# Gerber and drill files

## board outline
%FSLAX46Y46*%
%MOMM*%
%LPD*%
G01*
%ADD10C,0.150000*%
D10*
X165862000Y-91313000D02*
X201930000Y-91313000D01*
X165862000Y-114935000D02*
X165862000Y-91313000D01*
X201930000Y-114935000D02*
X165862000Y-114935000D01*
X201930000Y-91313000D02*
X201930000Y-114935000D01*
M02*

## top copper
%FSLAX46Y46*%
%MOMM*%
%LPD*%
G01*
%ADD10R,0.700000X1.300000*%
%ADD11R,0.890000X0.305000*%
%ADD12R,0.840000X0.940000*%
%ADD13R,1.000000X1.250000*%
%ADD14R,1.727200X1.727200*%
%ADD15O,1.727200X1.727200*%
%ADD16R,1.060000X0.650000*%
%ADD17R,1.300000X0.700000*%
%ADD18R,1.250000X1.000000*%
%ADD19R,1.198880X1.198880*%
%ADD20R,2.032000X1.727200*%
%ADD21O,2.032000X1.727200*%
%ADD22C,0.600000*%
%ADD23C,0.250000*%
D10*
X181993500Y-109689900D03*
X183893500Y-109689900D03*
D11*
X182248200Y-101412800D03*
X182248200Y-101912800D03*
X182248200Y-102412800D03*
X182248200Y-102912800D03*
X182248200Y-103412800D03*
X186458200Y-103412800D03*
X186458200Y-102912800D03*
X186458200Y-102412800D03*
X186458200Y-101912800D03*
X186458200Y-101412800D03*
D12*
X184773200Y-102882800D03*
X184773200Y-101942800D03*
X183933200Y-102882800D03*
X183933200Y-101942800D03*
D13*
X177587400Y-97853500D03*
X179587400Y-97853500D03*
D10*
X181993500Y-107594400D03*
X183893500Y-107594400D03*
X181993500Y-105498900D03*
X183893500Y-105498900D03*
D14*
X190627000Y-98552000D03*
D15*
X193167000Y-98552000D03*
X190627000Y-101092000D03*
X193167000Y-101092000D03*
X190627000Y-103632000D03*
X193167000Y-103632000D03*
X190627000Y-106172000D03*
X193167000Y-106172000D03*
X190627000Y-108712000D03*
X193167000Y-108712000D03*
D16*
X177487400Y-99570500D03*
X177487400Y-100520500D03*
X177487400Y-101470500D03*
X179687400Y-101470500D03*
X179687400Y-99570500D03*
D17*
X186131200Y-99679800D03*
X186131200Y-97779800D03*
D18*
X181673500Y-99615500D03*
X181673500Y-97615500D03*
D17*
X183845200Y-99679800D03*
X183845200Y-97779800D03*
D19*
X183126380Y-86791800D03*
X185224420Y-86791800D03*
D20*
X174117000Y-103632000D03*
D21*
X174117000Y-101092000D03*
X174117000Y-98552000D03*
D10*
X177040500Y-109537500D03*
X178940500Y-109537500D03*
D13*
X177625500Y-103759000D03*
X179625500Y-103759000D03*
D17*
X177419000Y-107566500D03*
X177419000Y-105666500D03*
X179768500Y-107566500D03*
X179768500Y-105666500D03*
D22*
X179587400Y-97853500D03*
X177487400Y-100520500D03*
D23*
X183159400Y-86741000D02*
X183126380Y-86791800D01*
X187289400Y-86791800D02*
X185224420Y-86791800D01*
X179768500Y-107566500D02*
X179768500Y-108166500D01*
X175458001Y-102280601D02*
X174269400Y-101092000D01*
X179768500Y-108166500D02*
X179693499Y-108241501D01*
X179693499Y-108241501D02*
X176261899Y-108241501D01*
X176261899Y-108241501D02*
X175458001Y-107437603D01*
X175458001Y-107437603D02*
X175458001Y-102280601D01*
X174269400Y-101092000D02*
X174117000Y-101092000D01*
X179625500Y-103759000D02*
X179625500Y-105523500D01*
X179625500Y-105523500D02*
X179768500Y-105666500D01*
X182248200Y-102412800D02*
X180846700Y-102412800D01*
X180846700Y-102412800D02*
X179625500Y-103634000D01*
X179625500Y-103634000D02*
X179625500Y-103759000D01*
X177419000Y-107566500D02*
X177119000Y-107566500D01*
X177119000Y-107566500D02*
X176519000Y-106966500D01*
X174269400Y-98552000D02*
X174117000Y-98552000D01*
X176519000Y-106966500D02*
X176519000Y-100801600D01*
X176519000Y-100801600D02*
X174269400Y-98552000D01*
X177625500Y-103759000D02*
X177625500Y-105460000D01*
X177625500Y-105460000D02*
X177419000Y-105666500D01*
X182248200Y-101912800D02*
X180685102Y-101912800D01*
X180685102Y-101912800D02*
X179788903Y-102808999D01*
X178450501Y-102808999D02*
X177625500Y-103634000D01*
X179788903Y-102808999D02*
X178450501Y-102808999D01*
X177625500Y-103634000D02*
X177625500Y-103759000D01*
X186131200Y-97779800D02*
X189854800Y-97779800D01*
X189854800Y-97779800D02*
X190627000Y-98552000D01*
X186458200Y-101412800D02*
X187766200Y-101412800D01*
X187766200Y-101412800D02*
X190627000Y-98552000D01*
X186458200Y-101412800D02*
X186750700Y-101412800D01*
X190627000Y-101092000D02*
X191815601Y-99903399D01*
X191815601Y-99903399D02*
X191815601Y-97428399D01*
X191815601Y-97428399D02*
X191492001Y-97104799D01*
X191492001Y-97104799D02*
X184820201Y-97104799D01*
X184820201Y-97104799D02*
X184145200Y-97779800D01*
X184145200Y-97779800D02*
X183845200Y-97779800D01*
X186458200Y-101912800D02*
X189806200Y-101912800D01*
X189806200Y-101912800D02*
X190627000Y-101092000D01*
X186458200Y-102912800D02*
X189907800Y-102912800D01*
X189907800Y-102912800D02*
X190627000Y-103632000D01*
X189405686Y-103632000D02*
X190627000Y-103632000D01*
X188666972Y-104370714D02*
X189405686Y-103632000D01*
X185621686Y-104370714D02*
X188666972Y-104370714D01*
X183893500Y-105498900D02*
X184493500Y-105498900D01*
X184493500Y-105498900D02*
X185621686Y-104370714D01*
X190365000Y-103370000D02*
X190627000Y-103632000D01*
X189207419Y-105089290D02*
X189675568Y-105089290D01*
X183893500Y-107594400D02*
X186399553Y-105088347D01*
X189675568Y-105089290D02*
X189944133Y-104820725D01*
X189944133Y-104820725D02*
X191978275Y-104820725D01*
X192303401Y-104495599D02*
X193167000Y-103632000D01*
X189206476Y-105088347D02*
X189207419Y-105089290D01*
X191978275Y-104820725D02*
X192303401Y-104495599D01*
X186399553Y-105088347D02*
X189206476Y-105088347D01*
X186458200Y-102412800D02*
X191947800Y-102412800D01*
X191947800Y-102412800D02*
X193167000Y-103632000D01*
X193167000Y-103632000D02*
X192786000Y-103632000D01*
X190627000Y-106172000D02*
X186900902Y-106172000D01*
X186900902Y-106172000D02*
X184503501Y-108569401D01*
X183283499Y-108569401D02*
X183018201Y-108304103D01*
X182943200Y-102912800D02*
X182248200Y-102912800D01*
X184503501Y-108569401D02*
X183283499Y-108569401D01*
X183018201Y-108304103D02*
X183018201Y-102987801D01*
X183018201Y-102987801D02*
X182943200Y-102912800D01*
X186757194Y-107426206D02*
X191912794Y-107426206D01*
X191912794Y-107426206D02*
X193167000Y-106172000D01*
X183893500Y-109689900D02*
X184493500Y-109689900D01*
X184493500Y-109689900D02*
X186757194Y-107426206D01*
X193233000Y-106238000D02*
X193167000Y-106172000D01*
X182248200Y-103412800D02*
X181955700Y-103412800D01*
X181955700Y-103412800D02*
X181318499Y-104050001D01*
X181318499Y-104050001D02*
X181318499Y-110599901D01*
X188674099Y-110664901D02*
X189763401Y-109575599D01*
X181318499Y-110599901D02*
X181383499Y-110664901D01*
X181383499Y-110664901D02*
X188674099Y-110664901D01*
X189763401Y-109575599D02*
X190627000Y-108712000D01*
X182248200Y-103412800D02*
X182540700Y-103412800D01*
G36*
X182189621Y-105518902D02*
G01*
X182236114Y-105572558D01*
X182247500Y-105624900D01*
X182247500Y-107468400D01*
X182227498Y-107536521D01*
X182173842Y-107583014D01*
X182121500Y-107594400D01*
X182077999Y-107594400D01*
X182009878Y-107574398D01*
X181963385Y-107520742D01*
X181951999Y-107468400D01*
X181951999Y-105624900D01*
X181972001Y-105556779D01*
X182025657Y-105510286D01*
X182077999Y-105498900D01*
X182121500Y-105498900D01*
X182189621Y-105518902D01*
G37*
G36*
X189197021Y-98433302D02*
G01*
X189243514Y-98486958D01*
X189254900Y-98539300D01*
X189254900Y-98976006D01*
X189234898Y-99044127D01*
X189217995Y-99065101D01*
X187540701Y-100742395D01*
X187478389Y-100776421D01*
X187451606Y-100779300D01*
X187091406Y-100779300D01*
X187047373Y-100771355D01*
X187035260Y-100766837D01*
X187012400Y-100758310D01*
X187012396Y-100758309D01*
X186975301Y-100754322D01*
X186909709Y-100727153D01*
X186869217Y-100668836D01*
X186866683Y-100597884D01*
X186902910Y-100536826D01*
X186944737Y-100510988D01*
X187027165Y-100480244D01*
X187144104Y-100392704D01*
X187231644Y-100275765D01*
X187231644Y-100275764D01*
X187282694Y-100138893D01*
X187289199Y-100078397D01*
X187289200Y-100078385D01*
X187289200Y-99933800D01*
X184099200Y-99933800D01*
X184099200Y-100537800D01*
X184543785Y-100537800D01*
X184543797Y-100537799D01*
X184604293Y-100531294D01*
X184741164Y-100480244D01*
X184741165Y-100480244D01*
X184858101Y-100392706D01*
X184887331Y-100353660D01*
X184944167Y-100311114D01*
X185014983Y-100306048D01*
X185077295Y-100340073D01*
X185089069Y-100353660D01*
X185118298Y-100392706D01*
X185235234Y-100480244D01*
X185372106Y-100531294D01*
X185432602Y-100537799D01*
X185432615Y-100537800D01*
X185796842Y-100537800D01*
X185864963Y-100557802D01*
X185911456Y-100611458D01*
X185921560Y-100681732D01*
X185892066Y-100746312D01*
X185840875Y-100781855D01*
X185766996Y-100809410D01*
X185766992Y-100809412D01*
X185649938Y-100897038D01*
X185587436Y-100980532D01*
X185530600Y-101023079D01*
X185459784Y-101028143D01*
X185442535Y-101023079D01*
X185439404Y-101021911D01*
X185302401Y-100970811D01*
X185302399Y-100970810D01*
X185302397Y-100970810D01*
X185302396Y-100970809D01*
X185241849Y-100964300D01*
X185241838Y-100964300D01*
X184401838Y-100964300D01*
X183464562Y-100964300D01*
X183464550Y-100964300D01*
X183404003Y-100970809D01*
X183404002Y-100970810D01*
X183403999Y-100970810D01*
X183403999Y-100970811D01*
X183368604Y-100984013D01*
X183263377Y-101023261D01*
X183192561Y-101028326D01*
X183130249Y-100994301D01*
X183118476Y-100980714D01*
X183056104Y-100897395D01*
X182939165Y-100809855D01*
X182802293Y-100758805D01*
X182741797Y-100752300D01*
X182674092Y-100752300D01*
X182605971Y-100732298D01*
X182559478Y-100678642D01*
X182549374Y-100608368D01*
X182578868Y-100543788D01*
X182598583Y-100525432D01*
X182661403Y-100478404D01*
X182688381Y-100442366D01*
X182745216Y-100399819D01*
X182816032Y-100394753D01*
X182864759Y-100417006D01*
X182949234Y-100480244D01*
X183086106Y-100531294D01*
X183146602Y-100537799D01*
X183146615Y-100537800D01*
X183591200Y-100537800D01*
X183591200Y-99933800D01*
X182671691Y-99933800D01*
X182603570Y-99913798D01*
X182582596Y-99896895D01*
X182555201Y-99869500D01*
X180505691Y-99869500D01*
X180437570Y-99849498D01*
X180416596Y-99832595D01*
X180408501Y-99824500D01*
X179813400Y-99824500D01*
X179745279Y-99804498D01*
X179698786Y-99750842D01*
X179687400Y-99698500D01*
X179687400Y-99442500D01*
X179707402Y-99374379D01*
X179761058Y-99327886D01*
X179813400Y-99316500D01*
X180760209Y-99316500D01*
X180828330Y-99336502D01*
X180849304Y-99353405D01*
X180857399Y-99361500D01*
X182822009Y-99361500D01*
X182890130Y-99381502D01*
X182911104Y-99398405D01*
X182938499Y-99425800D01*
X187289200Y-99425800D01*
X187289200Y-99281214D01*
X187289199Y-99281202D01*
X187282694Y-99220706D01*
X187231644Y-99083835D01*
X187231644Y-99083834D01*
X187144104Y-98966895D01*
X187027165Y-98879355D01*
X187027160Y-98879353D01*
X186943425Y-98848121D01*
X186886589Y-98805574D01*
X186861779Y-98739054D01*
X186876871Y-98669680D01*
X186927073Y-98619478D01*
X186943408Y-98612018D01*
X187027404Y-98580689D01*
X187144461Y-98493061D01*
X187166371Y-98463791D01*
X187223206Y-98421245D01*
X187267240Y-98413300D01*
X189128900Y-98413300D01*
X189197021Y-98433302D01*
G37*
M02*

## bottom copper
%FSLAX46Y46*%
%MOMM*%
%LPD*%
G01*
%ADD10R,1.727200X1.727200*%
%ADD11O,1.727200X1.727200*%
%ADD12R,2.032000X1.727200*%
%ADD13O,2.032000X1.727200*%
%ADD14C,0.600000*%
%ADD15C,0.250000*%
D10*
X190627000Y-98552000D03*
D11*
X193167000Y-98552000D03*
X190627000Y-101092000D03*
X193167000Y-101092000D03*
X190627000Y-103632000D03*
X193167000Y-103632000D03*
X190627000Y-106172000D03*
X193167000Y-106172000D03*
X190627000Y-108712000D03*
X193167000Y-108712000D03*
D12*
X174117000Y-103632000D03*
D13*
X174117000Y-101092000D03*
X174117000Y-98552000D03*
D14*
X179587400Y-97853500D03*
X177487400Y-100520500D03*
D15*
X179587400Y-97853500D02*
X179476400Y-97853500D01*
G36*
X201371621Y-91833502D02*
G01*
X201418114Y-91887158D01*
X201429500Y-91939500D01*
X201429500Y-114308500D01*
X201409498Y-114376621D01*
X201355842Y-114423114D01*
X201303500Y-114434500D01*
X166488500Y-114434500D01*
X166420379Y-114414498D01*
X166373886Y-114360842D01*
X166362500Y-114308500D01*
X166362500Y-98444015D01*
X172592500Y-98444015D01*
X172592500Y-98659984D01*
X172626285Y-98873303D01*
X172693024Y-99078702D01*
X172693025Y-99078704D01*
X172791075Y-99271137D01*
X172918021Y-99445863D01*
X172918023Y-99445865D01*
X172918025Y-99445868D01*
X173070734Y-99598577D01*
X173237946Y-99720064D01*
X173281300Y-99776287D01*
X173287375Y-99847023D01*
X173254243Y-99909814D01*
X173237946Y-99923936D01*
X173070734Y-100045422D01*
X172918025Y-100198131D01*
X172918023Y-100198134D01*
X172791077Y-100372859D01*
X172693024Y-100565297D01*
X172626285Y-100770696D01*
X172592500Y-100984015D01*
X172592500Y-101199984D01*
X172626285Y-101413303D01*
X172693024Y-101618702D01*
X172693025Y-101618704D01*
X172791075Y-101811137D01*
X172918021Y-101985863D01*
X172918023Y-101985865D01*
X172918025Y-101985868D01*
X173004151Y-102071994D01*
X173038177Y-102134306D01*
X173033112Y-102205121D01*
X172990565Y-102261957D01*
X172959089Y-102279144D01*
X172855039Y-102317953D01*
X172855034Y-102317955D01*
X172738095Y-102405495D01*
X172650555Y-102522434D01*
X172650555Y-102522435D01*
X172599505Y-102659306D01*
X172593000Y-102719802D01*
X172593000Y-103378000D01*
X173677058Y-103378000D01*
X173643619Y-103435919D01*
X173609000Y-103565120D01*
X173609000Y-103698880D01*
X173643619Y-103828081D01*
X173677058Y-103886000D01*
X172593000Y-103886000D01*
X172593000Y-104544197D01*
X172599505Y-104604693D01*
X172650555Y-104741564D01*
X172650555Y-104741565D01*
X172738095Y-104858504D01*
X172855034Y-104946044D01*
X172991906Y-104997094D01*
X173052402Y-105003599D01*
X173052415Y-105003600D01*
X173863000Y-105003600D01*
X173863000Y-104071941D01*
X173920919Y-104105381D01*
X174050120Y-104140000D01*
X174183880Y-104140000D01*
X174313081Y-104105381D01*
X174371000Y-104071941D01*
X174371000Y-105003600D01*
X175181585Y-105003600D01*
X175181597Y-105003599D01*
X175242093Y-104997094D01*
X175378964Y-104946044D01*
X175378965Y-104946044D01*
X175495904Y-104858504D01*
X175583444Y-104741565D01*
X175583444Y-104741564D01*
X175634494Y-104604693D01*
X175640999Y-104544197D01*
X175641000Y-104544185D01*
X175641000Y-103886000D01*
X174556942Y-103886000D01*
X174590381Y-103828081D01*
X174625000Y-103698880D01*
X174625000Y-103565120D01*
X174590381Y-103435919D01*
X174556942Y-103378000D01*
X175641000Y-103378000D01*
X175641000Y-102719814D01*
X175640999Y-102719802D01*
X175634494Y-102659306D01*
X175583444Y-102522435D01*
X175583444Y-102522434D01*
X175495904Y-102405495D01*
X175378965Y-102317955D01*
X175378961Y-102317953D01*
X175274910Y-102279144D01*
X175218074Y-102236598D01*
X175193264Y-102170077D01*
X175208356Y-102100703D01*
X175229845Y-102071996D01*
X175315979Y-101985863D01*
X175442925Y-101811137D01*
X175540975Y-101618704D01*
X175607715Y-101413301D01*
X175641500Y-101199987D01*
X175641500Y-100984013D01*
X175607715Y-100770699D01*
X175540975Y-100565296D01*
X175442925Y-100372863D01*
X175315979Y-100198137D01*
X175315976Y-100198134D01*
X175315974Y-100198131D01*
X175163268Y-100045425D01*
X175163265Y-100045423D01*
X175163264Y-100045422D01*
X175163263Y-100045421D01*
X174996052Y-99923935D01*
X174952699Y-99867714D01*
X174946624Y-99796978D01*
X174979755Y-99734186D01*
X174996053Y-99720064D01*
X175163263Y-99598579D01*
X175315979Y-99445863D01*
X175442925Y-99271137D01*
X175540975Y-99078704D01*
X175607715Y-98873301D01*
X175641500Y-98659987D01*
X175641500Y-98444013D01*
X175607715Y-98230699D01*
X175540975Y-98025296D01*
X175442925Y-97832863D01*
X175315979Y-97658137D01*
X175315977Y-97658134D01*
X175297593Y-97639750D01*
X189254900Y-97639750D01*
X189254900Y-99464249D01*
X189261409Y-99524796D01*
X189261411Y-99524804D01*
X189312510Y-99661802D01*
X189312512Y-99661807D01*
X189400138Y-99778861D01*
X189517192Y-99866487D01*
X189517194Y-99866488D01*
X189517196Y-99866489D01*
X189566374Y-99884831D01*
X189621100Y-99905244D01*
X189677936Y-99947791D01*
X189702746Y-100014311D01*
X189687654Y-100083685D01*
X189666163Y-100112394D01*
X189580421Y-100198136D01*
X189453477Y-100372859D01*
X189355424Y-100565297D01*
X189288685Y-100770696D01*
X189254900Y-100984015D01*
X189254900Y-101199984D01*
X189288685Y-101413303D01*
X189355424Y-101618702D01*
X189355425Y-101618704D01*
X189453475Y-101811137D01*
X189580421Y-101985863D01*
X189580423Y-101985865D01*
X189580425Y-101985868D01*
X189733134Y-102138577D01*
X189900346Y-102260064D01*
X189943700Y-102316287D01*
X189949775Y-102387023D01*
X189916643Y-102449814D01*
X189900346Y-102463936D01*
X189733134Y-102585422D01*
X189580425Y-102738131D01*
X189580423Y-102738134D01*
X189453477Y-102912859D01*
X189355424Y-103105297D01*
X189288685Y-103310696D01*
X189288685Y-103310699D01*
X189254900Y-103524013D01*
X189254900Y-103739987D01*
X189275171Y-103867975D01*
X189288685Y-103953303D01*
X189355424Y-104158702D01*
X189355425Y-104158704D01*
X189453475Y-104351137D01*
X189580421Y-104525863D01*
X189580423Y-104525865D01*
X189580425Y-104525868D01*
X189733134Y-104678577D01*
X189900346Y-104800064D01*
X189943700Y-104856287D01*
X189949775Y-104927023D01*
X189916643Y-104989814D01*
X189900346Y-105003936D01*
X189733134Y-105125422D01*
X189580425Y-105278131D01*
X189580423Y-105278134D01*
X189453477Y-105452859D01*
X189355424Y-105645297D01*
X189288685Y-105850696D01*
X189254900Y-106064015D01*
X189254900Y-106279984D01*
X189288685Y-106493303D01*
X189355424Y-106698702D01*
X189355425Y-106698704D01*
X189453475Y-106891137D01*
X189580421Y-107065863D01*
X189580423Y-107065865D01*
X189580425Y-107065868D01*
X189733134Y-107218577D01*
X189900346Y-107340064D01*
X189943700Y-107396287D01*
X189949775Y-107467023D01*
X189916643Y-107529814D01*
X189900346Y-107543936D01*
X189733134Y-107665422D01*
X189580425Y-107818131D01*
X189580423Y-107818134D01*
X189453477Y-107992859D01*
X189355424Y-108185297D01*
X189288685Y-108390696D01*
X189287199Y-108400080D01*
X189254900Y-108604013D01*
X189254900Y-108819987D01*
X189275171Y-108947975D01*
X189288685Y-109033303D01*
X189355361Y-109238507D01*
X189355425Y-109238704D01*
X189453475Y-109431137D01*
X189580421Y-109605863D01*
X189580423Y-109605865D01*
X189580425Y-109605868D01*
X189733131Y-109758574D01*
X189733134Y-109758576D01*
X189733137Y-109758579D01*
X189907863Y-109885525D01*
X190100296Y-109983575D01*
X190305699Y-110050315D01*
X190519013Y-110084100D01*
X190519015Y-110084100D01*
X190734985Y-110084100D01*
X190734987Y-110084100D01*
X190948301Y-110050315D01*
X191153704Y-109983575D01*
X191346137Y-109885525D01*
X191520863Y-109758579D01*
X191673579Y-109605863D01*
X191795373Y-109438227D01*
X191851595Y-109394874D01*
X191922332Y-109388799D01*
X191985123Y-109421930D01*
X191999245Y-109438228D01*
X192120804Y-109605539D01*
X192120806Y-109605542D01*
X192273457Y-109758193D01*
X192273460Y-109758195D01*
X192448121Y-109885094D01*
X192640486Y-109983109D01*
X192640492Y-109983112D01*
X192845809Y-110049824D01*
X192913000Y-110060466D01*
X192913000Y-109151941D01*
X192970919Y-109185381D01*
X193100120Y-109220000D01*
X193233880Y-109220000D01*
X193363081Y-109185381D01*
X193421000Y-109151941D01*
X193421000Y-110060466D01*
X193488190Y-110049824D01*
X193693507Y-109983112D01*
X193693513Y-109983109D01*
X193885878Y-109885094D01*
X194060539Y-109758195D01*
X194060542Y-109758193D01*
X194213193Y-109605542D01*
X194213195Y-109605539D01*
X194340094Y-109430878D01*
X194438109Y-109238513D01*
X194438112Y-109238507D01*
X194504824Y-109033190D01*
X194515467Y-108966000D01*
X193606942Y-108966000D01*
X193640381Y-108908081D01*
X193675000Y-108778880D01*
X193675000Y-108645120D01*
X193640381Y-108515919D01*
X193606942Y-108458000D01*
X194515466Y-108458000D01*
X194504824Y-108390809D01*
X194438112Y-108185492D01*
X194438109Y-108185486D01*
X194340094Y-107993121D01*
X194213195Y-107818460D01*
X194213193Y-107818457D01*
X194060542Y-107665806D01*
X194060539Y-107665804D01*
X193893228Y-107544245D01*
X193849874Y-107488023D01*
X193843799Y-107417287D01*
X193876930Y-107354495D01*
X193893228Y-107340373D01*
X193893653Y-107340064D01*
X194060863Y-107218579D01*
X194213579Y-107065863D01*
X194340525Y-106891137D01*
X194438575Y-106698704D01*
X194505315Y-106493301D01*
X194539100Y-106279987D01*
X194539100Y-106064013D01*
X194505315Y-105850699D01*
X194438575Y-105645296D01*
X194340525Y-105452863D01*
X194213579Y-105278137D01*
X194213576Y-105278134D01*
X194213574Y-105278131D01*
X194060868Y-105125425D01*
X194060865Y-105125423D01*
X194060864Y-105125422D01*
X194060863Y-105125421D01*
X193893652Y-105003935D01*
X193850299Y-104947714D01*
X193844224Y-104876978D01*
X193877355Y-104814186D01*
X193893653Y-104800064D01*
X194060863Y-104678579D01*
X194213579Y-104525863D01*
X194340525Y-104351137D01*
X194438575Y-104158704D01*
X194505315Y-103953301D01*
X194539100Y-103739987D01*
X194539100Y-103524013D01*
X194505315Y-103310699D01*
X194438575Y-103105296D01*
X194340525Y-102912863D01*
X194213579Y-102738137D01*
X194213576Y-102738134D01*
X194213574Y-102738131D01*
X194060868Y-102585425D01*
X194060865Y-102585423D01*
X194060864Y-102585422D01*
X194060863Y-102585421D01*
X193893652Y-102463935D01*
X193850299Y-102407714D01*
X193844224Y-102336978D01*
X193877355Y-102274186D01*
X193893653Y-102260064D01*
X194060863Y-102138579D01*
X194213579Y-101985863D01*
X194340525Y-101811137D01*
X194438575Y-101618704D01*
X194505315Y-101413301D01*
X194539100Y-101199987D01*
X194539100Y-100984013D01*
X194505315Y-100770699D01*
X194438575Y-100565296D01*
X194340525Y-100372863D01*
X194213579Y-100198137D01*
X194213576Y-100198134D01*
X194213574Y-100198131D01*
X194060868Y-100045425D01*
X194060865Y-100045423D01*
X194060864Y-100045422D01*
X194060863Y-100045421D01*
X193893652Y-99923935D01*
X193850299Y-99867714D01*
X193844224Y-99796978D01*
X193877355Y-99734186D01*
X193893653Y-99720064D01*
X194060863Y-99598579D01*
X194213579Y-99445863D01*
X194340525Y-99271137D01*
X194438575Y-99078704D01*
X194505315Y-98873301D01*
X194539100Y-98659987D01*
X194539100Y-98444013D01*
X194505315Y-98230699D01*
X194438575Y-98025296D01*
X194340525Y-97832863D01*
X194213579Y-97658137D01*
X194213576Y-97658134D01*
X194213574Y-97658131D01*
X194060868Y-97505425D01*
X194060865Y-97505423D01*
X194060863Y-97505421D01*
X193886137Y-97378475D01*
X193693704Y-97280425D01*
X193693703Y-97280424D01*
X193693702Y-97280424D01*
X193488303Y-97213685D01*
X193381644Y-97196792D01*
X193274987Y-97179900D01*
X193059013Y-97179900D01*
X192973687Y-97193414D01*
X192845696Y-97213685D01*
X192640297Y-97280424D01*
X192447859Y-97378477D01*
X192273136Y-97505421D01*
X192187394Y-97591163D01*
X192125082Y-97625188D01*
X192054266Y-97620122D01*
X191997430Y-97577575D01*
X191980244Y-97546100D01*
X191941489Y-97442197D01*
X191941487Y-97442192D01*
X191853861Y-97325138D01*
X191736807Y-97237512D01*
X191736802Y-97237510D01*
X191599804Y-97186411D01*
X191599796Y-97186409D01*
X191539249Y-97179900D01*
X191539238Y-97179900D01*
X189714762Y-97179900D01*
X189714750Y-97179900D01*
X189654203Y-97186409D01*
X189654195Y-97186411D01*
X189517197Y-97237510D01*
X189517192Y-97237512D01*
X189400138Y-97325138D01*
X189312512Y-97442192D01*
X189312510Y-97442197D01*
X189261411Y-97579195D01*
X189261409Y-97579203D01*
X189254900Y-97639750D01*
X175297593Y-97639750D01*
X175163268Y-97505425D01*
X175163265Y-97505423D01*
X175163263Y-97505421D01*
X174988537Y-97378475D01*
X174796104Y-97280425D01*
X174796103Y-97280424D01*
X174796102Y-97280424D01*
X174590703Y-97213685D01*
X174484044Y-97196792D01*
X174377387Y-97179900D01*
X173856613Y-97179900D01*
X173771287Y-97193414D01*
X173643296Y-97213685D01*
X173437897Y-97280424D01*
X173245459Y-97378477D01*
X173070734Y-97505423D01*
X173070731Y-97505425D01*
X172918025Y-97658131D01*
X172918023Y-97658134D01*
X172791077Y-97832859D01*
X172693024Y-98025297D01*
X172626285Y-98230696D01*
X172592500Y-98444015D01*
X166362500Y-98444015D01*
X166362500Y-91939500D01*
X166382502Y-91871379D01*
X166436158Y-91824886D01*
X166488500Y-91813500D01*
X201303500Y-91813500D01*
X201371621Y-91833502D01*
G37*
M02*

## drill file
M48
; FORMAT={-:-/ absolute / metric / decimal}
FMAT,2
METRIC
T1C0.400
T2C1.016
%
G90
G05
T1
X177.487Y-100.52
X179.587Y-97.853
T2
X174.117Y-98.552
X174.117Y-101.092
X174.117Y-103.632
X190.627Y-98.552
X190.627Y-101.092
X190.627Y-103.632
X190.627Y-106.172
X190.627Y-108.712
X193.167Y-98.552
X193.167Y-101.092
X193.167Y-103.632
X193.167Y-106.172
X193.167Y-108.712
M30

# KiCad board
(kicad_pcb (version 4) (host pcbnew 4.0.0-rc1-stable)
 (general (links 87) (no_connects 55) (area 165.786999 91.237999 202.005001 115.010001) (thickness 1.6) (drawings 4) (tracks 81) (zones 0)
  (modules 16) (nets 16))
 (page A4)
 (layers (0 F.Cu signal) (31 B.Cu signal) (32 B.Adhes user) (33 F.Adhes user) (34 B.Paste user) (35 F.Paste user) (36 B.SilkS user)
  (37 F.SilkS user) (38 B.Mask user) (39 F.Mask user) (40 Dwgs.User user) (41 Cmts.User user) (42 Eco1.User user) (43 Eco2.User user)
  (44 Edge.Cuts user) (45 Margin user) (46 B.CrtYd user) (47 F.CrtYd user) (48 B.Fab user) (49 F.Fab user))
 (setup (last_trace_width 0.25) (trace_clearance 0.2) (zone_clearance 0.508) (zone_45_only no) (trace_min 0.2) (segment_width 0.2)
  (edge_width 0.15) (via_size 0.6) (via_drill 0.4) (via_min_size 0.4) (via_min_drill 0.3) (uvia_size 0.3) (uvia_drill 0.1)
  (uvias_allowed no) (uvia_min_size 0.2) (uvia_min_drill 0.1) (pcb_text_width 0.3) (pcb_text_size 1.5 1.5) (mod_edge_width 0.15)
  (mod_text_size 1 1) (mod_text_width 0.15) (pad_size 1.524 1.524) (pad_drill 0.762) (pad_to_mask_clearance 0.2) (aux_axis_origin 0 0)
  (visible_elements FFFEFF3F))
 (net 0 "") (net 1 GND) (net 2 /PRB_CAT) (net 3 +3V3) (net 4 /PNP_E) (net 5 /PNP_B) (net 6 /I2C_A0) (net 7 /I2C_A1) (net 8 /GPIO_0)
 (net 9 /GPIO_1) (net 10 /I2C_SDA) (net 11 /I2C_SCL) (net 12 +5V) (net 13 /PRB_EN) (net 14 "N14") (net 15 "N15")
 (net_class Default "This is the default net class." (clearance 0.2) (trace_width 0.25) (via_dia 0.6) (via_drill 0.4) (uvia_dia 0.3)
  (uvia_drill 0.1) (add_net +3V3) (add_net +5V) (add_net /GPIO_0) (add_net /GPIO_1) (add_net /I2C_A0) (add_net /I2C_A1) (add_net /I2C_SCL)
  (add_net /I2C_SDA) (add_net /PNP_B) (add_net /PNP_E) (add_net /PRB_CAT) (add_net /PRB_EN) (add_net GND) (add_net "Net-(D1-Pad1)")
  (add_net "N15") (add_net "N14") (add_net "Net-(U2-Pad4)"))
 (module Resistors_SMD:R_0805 (layer F.Cu) (at 182.9435 109.6899)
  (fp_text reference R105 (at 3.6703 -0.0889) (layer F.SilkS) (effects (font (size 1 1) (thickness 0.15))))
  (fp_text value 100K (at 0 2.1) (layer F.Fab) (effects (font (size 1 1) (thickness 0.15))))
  (pad 1 smd rect (at -0.95 0) (size 0.7 1.3) (layers F.Cu F.Paste F.Mask) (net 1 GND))
  (pad 2 smd rect (at 0.95 0) (size 0.7 1.3) (layers F.Cu F.Paste F.Mask) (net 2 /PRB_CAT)))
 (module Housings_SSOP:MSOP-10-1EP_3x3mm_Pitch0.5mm (layer F.Cu) (at 184.3532 102.4128)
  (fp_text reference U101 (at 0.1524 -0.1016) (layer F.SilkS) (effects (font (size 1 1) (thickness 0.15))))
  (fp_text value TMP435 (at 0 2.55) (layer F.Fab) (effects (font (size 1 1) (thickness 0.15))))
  (pad 1 smd rect (at -2.105 -1) (size 0.89 0.305) (layers F.Cu F.Paste F.Mask) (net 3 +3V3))
  (pad 2 smd rect (at -2.105 -0.5) (size 0.89 0.305) (layers F.Cu F.Paste F.Mask) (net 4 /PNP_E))
  (pad 3 smd rect (at -2.105 0) (size 0.89 0.305) (layers F.Cu F.Paste F.Mask) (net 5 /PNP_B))
  (pad 4 smd rect (at -2.105 0.5) (size 0.89 0.305) (layers F.Cu F.Paste F.Mask) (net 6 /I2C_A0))
  (pad 5 smd rect (at -2.105 1) (size 0.89 0.305) (layers F.Cu F.Paste F.Mask) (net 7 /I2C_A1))
  (pad 6 smd rect (at 2.105 1) (size 0.89 0.305) (layers F.Cu F.Paste F.Mask) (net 1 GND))
  (pad 7 smd rect (at 2.105 0.5) (size 0.89 0.305) (layers F.Cu F.Paste F.Mask) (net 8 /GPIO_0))
  (pad 8 smd rect (at 2.105 0) (size 0.89 0.305) (layers F.Cu F.Paste F.Mask) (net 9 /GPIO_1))
  (pad 9 smd rect (at 2.105 -0.5) (size 0.89 0.305) (layers F.Cu F.Paste F.Mask) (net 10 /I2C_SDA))
  (pad 10 smd rect (at 2.105 -1) (size 0.89 0.305) (layers F.Cu F.Paste F.Mask) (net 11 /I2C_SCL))
  (pad 11 smd rect (at 0.42 0.47) (size 0.84 0.94) (layers F.Cu F.Paste F.Mask) (solder_paste_margin_ratio -0.2))
  (pad 11 smd rect (at 0.42 -0.47) (size 0.84 0.94) (layers F.Cu F.Paste F.Mask) (solder_paste_margin_ratio -0.2))
  (pad 11 smd rect (at -0.42 0.47) (size 0.84 0.94) (layers F.Cu F.Paste F.Mask) (solder_paste_margin_ratio -0.2))
  (pad 11 smd rect (at -0.42 -0.47) (size 0.84 0.94) (layers F.Cu F.Paste F.Mask) (solder_paste_margin_ratio -0.2)))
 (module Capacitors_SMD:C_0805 (layer F.Cu) (at 178.5874 97.8535)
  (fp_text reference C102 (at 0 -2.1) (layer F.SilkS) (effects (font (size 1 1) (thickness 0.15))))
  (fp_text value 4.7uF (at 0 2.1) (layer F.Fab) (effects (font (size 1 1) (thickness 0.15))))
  (pad 1 smd rect (at -1 0) (size 1 1.25) (layers F.Cu F.Paste F.Mask) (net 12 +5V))
  (pad 2 smd rect (at 1 0) (size 1 1.25) (layers F.Cu F.Paste F.Mask) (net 1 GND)))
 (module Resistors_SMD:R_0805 (layer F.Cu) (at 182.9435 107.5944)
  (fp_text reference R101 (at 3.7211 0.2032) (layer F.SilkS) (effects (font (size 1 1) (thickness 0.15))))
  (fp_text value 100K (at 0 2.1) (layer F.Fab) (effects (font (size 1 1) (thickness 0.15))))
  (pad 1 smd rect (at -0.95 0) (size 0.7 1.3) (layers F.Cu F.Paste F.Mask) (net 3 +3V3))
  (pad 2 smd rect (at 0.95 0) (size 0.7 1.3) (layers F.Cu F.Paste F.Mask) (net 9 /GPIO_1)))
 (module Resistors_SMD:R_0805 (layer F.Cu) (at 182.9435 105.4989)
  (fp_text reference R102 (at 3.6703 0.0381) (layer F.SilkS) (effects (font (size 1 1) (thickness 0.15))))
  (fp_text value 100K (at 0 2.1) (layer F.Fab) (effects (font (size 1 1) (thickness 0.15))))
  (pad 1 smd rect (at -0.95 0) (size 0.7 1.3) (layers F.Cu F.Paste F.Mask) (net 3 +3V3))
  (pad 2 smd rect (at 0.95 0) (size 0.7 1.3) (layers F.Cu F.Paste F.Mask) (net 8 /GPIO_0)))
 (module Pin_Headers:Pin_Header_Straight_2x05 (layer F.Cu) (at 190.627 98.552)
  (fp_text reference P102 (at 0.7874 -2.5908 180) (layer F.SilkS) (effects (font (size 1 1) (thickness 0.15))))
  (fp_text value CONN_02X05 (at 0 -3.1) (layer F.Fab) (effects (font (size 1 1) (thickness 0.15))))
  (pad 1 thru_hole rect (at 0 0) (size 1.7272 1.7272) (drill 1.016) (layers *.Cu *.Mask F.SilkS) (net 11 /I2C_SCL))
  (pad 2 thru_hole oval (at 2.54 0) (size 1.7272 1.7272) (drill 1.016) (layers *.Cu *.Mask F.SilkS) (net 12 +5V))
  (pad 3 thru_hole oval (at 0 2.54) (size 1.7272 1.7272) (drill 1.016) (layers *.Cu *.Mask F.SilkS) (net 10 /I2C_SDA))
  (pad 4 thru_hole oval (at 2.54 2.54) (size 1.7272 1.7272) (drill 1.016) (layers *.Cu *.Mask F.SilkS) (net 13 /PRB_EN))
  (pad 5 thru_hole oval (at 0 5.08) (size 1.7272 1.7272) (drill 1.016) (layers *.Cu *.Mask F.SilkS) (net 8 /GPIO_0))
  (pad 6 thru_hole oval (at 2.54 5.08) (size 1.7272 1.7272) (drill 1.016) (layers *.Cu *.Mask F.SilkS) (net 9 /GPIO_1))
  (pad 7 thru_hole oval (at 0 7.62) (size 1.7272 1.7272) (drill 1.016) (layers *.Cu *.Mask F.SilkS) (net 6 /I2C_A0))
  (pad 8 thru_hole oval (at 2.54 7.62) (size 1.7272 1.7272) (drill 1.016) (layers *.Cu *.Mask F.SilkS) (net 2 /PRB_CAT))
  (pad 9 thru_hole oval (at 0 10.16) (size 1.7272 1.7272) (drill 1.016) (layers *.Cu *.Mask F.SilkS) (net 7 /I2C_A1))
  (pad 10 thru_hole oval (at 2.54 10.16) (size 1.7272 1.7272) (drill 1.016) (layers *.Cu *.Mask F.SilkS) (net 1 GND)))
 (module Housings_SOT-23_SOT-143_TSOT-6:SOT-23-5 (layer F.Cu) (at 178.5874 100.5205)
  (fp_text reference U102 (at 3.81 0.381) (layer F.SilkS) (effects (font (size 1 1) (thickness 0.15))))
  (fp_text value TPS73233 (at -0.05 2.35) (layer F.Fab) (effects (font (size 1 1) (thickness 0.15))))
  (pad 1 smd rect (at -1.1 -0.95) (size 1.06 0.65) (layers F.Cu F.Paste F.Mask) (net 12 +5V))
  (pad 2 smd rect (at -1.1 0) (size 1.06 0.65) (layers F.Cu F.Paste F.Mask) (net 1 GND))
  (pad 3 smd rect (at -1.1 0.95) (size 1.06 0.65) (layers F.Cu F.Paste F.Mask) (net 13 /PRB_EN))
  (pad 4 smd rect (at 1.1 0.95) (size 1.06 0.65) (layers F.Cu F.Paste F.Mask) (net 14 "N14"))
  (pad 5 smd rect (at 1.1 -0.95) (size 1.06 0.65) (layers F.Cu F.Paste F.Mask) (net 3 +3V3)))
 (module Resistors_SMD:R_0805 (layer F.Cu) (at 186.1312 98.7298 90)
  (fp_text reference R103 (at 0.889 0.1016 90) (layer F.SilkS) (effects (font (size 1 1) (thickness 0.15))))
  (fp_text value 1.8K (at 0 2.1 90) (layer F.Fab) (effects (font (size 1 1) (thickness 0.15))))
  (pad 1 smd rect (at -0.95 0 90) (size 0.7 1.3) (layers F.Cu F.Paste F.Mask) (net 3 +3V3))
  (pad 2 smd rect (at 0.95 0 90) (size 0.7 1.3) (layers F.Cu F.Paste F.Mask) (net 11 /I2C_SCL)))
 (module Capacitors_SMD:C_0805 (layer F.Cu) (at 181.6735 98.6155 90)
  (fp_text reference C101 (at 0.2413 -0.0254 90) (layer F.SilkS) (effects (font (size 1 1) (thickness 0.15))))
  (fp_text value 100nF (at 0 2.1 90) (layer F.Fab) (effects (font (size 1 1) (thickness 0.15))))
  (pad 1 smd rect (at -1 0 90) (size 1 1.25) (layers F.Cu F.Paste F.Mask) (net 3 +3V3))
  (pad 2 smd rect (at 1 0 90) (size 1 1.25) (layers F.Cu F.Paste F.Mask) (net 1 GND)))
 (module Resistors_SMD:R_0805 (layer F.Cu) (at 183.8452 98.7298 90)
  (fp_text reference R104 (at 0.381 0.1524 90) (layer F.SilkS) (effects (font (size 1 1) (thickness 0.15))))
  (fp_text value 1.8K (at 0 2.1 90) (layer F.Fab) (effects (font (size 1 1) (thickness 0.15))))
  (pad 1 smd rect (at -0.95 0 90) (size 0.7 1.3) (layers F.Cu F.Paste F.Mask) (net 3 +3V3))
  (pad 2 smd rect (at 0.95 0 90) (size 0.7 1.3) (layers F.Cu F.Paste F.Mask) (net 10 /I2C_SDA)))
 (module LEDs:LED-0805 (layer F.Cu) (at 184.1754 86.7918 180)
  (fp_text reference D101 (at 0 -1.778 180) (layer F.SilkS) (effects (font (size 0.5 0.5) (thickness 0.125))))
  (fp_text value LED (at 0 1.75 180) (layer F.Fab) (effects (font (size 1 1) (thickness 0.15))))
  (pad 2 smd rect (at 1.04902 0) (size 1.19888 1.19888) (layers F.Cu F.Paste F.Mask) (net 3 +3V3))
  (pad 1 smd rect (at -1.04902 0) (size 1.19888 1.19888) (layers F.Cu F.Paste F.Mask) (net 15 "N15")))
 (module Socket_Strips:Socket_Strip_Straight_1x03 (layer F.Cu) (at 174.117 103.632 90)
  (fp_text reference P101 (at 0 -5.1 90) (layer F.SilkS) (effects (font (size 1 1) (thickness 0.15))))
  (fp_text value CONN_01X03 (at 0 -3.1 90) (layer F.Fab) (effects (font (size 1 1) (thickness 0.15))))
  (pad 1 thru_hole rect (at 0 0 90) (size 1.7272 2.032) (drill 1.016) (layers *.Cu *.Mask F.SilkS) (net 1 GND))
  (pad 2 thru_hole oval (at 2.54 0 90) (size 1.7272 2.032) (drill 1.016) (layers *.Cu *.Mask F.SilkS) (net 5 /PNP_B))
  (pad 3 thru_hole oval (at 5.08 0 90) (size 1.7272 2.032) (drill 1.016) (layers *.Cu *.Mask F.SilkS) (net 4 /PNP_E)))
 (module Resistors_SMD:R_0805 (layer F.Cu) (at 177.9905 109.5375)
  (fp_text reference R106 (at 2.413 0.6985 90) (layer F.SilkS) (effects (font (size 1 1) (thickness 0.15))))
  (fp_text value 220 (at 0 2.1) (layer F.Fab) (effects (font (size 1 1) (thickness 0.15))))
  (pad 1 smd rect (at -0.95 0) (size 0.7 1.3) (layers F.Cu F.Paste F.Mask) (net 15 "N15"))
  (pad 2 smd rect (at 0.95 0) (size 0.7 1.3) (layers F.Cu F.Paste F.Mask) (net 1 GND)))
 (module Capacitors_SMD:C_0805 (layer F.Cu) (at 178.6255 103.759)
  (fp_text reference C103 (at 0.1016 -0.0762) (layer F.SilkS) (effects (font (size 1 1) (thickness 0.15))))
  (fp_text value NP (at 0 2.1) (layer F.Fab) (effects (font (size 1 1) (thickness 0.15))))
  (pad 1 smd rect (at -1 0) (size 1 1.25) (layers F.Cu F.Paste F.Mask) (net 4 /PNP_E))
  (pad 2 smd rect (at 1 0) (size 1 1.25) (layers F.Cu F.Paste F.Mask) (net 5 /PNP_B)))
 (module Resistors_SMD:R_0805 (layer F.Cu) (at 177.419 106.6165 90)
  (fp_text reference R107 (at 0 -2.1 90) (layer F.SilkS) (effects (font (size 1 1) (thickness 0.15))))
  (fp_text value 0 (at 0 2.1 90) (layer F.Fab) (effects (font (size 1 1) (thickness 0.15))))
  (pad 1 smd rect (at -0.95 0 90) (size 0.7 1.3) (layers F.Cu F.Paste F.Mask) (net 4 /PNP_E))
  (pad 2 smd rect (at 0.95 0 90) (size 0.7 1.3) (layers F.Cu F.Paste F.Mask) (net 4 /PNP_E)))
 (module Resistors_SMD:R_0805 (layer F.Cu) (at 179.7685 106.6165 90)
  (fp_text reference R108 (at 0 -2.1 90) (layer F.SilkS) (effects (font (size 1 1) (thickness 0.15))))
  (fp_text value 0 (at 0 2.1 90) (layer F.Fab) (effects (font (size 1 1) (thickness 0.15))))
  (pad 1 smd rect (at -0.95 0 90) (size 0.7 1.3) (layers F.Cu F.Paste F.Mask) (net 5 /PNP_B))
  (pad 2 smd rect (at 0.95 0 90) (size 0.7 1.3) (layers F.Cu F.Paste F.Mask) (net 5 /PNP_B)))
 (gr_line (start 165.862 91.313) (end 201.93 91.313) (angle 90) (layer Edge.Cuts) (width 0.15))
 (gr_line (start 165.862 114.935) (end 165.862 91.313) (angle 90) (layer Edge.Cuts) (width 0.15))
 (gr_line (start 201.93 114.935) (end 165.862 114.935) (angle 90) (layer Edge.Cuts) (width 0.15))
 (gr_line (start 201.93 91.313) (end 201.93 114.935) (angle 90) (layer Edge.Cuts) (width 0.15))
 (segment (start 183.1594 86.741) (end 183.12638 86.7918) (width 0.25) (layer F.Cu) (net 3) (status 80000))
 (via (at 179.5874 97.8535) (size 0.6) (drill 0.4) (layers F.Cu B.Cu) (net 1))
 (via (at 177.4874 100.5205) (size 0.6) (drill 0.4) (layers F.Cu B.Cu) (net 1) (status 30))
 (segment (start 179.5874 97.8535) (end 179.4764 97.8535) (width 0.25) (layer B.Cu) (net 1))
 (segment (start 187.2894 86.7918) (end 185.22442 86.7918) (width 0.25) (layer F.Cu) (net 15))
 (segment (start 179.7685 107.5665) (end 179.7685 108.1665) (width 0.25) (layer F.Cu) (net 5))
 (segment (start 175.458001 102.280601) (end 174.2694 101.092) (width 0.25) (layer F.Cu) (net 5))
 (segment (start 179.7685 108.1665) (end 179.693499 108.241501) (width 0.25) (layer F.Cu) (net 5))
 (segment (start 179.693499 108.241501) (end 176.261899 108.241501) (width 0.25) (layer F.Cu) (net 5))
 (segment (start 176.261899 108.241501) (end 175.458001 107.437603) (width 0.25) (layer F.Cu) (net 5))
 (segment (start 175.458001 107.437603) (end 175.458001 102.280601) (width 0.25) (layer F.Cu) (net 5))
 (segment (start 174.2694 101.092) (end 174.117 101.092) (width 0.25) (layer F.Cu) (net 5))
 (segment (start 179.6255 103.759) (end 179.6255 105.5235) (width 0.25) (layer F.Cu) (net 5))
 (segment (start 179.6255 105.5235) (end 179.7685 105.6665) (width 0.25) (layer F.Cu) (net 5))
 (segment (start 182.2482 102.4128) (end 180.8467 102.4128) (width 0.25) (layer F.Cu) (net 5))
 (segment (start 180.8467 102.4128) (end 179.6255 103.634) (width 0.25) (layer F.Cu) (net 5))
 (segment (start 179.6255 103.634) (end 179.6255 103.759) (width 0.25) (layer F.Cu) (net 5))
 (segment (start 177.419 107.5665) (end 177.119 107.5665) (width 0.25) (layer F.Cu) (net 4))
 (segment (start 177.119 107.5665) (end 176.519 106.9665) (width 0.25) (layer F.Cu) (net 4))
 (segment (start 174.2694 98.552) (end 174.117 98.552) (width 0.25) (layer F.Cu) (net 4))
 (segment (start 176.519 106.9665) (end 176.519 100.8016) (width 0.25) (layer F.Cu) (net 4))
 (segment (start 176.519 100.8016) (end 174.2694 98.552) (width 0.25) (layer F.Cu) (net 4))
 (segment (start 177.6255 103.759) (end 177.6255 105.46) (width 0.25) (layer F.Cu) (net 4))
 (segment (start 177.6255 105.46) (end 177.419 105.6665) (width 0.25) (layer F.Cu) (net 4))
 (segment (start 182.2482 101.9128) (end 180.685102 101.9128) (width 0.25) (layer F.Cu) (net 4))
 (segment (start 180.685102 101.9128) (end 179.788903 102.808999) (width 0.25) (layer F.Cu) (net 4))
 (segment (start 178.450501 102.808999) (end 177.6255 103.634) (width 0.25) (layer F.Cu) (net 4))
 (segment (start 179.788903 102.808999) (end 178.450501 102.808999) (width 0.25) (layer F.Cu) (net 4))
 (segment (start 177.6255 103.634) (end 177.6255 103.759) (width 0.25) (layer F.Cu) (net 4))
 (segment (start 186.1312 97.7798) (end 189.8548 97.7798) (width 0.25) (layer F.Cu) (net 11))
 (segment (start 189.8548 97.7798) (end 190.627 98.552) (width 0.25) (layer F.Cu) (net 11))
 (segment (start 186.4582 101.4128) (end 187.7662 101.4128) (width 0.25) (layer F.Cu) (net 11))
 (segment (start 187.7662 101.4128) (end 190.627 98.552) (width 0.25) (layer F.Cu) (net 11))
 (segment (start 186.4582 101.4128) (end 186.7507 101.4128) (width 0.25) (layer F.Cu) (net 11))
 (segment (start 190.627 101.092) (end 191.815601 99.903399) (width 0.25) (layer F.Cu) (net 10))
 (segment (start 191.815601 99.903399) (end 191.815601 97.428399) (width 0.25) (layer F.Cu) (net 10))
 (segment (start 191.815601 97.428399) (end 191.492001 97.104799) (width 0.25) (layer F.Cu) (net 10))
 (segment (start 191.492001 97.104799) (end 184.820201 97.104799) (width 0.25) (layer F.Cu) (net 10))
 (segment (start 184.820201 97.104799) (end 184.1452 97.7798) (width 0.25) (layer F.Cu) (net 10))
 (segment (start 184.1452 97.7798) (end 183.8452 97.7798) (width 0.25) (layer F.Cu) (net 10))
 (segment (start 186.4582 101.9128) (end 189.8062 101.9128) (width 0.25) (layer F.Cu) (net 10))
 (segment (start 189.8062 101.9128) (end 190.627 101.092) (width 0.25) (layer F.Cu) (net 10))
 (segment (start 186.4582 102.9128) (end 189.9078 102.9128) (width 0.25) (layer F.Cu) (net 8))
 (segment (start 189.9078 102.9128) (end 190.627 103.632) (width 0.25) (layer F.Cu) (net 8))
 (segment (start 189.405686 103.632) (end 190.627 103.632) (width 0.25) (layer F.Cu) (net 8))
 (segment (start 188.666972 104.370714) (end 189.405686 103.632) (width 0.25) (layer F.Cu) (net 8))
 (segment (start 185.621686 104.370714) (end 188.666972 104.370714) (width 0.25) (layer F.Cu) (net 8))
 (segment (start 183.8935 105.4989) (end 184.4935 105.4989) (width 0.25) (layer F.Cu) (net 8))
 (segment (start 184.4935 105.4989) (end 185.621686 104.370714) (width 0.25) (layer F.Cu) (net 8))
 (segment (start 190.365 103.37) (end 190.627 103.632) (width 0.25) (layer F.Cu) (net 8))
 (segment (start 189.207419 105.08929) (end 189.675568 105.08929) (width 0.25) (layer F.Cu) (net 9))
 (segment (start 183.8935 107.5944) (end 186.399553 105.088347) (width 0.25) (layer F.Cu) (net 9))
 (segment (start 189.675568 105.08929) (end 189.944133 104.820725) (width 0.25) (layer F.Cu) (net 9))
 (segment (start 189.944133 104.820725) (end 191.978275 104.820725) (width 0.25) (layer F.Cu) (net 9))
 (segment (start 192.303401 104.495599) (end 193.167 103.632) (width 0.25) (layer F.Cu) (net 9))
 (segment (start 189.206476 105.088347) (end 189.207419 105.08929) (width 0.25) (layer F.Cu) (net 9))
 (segment (start 191.978275 104.820725) (end 192.303401 104.495599) (width 0.25) (layer F.Cu) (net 9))
 (segment (start 186.399553 105.088347) (end 189.206476 105.088347) (width 0.25) (layer F.Cu) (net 9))
 (segment (start 186.4582 102.4128) (end 191.9478 102.4128) (width 0.25) (layer F.Cu) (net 9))
 (segment (start 191.9478 102.4128) (end 193.167 103.632) (width 0.25) (layer F.Cu) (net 9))
 (segment (start 193.167 103.632) (end 192.786 103.632) (width 0.25) (layer F.Cu) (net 9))
 (segment (start 190.627 106.172) (end 186.900902 106.172) (width 0.25) (layer F.Cu) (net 6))
 (segment (start 186.900902 106.172) (end 184.503501 108.569401) (width 0.25) (layer F.Cu) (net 6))
 (segment (start 183.283499 108.569401) (end 183.018201 108.304103) (width 0.25) (layer F.Cu) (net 6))
 (segment (start 182.9432 102.9128) (end 182.2482 102.9128) (width 0.25) (layer F.Cu) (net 6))
 (segment (start 184.503501 108.569401) (end 183.283499 108.569401) (width 0.25) (layer F.Cu) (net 6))
 (segment (start 183.018201 108.304103) (end 183.018201 102.987801) (width 0.25) (layer F.Cu) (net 6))
 (segment (start 183.018201 102.987801) (end 182.9432 102.9128) (width 0.25) (layer F.Cu) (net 6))
 (segment (start 186.757194 107.426206) (end 191.912794 107.426206) (width 0.25) (layer F.Cu) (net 2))
 (segment (start 191.912794 107.426206) (end 193.167 106.172) (width 0.25) (layer F.Cu) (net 2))
 (segment (start 183.8935 109.6899) (end 184.4935 109.6899) (width 0.25) (layer F.Cu) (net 2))
 (segment (start 184.4935 109.6899) (end 186.757194 107.426206) (width 0.25) (layer F.Cu) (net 2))
 (segment (start 193.233 106.238) (end 193.167 106.172) (width 0.25) (layer F.Cu) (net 2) (status 30))
 (segment (start 182.2482 103.4128) (end 181.9557 103.4128) (width 0.25) (layer F.Cu) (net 7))
 (segment (start 181.9557 103.4128) (end 181.318499 104.050001) (width 0.25) (layer F.Cu) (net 7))
 (segment (start 181.318499 104.050001) (end 181.318499 110.599901) (width 0.25) (layer F.Cu) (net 7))
 (segment (start 188.674099 110.664901) (end 189.763401 109.575599) (width 0.25) (layer F.Cu) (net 7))
 (segment (start 181.318499 110.599901) (end 181.383499 110.664901) (width 0.25) (layer F.Cu) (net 7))
 (segment (start 181.383499 110.664901) (end 188.674099 110.664901) (width 0.25) (layer F.Cu) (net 7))
 (segment (start 189.763401 109.575599) (end 190.627 108.712) (width 0.25) (layer F.Cu) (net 7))
 (segment (start 182.2482 103.4128) (end 182.5407 103.4128) (width 0.25) (layer F.Cu) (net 7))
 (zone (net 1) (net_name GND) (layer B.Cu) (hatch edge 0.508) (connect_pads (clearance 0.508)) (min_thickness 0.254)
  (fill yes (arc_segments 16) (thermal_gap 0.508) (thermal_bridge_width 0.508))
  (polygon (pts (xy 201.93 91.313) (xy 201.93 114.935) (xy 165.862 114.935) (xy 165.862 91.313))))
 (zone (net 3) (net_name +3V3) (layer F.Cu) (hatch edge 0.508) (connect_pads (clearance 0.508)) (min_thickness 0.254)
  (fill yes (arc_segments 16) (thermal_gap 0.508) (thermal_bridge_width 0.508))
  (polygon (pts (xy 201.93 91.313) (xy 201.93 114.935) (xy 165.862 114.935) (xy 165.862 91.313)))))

